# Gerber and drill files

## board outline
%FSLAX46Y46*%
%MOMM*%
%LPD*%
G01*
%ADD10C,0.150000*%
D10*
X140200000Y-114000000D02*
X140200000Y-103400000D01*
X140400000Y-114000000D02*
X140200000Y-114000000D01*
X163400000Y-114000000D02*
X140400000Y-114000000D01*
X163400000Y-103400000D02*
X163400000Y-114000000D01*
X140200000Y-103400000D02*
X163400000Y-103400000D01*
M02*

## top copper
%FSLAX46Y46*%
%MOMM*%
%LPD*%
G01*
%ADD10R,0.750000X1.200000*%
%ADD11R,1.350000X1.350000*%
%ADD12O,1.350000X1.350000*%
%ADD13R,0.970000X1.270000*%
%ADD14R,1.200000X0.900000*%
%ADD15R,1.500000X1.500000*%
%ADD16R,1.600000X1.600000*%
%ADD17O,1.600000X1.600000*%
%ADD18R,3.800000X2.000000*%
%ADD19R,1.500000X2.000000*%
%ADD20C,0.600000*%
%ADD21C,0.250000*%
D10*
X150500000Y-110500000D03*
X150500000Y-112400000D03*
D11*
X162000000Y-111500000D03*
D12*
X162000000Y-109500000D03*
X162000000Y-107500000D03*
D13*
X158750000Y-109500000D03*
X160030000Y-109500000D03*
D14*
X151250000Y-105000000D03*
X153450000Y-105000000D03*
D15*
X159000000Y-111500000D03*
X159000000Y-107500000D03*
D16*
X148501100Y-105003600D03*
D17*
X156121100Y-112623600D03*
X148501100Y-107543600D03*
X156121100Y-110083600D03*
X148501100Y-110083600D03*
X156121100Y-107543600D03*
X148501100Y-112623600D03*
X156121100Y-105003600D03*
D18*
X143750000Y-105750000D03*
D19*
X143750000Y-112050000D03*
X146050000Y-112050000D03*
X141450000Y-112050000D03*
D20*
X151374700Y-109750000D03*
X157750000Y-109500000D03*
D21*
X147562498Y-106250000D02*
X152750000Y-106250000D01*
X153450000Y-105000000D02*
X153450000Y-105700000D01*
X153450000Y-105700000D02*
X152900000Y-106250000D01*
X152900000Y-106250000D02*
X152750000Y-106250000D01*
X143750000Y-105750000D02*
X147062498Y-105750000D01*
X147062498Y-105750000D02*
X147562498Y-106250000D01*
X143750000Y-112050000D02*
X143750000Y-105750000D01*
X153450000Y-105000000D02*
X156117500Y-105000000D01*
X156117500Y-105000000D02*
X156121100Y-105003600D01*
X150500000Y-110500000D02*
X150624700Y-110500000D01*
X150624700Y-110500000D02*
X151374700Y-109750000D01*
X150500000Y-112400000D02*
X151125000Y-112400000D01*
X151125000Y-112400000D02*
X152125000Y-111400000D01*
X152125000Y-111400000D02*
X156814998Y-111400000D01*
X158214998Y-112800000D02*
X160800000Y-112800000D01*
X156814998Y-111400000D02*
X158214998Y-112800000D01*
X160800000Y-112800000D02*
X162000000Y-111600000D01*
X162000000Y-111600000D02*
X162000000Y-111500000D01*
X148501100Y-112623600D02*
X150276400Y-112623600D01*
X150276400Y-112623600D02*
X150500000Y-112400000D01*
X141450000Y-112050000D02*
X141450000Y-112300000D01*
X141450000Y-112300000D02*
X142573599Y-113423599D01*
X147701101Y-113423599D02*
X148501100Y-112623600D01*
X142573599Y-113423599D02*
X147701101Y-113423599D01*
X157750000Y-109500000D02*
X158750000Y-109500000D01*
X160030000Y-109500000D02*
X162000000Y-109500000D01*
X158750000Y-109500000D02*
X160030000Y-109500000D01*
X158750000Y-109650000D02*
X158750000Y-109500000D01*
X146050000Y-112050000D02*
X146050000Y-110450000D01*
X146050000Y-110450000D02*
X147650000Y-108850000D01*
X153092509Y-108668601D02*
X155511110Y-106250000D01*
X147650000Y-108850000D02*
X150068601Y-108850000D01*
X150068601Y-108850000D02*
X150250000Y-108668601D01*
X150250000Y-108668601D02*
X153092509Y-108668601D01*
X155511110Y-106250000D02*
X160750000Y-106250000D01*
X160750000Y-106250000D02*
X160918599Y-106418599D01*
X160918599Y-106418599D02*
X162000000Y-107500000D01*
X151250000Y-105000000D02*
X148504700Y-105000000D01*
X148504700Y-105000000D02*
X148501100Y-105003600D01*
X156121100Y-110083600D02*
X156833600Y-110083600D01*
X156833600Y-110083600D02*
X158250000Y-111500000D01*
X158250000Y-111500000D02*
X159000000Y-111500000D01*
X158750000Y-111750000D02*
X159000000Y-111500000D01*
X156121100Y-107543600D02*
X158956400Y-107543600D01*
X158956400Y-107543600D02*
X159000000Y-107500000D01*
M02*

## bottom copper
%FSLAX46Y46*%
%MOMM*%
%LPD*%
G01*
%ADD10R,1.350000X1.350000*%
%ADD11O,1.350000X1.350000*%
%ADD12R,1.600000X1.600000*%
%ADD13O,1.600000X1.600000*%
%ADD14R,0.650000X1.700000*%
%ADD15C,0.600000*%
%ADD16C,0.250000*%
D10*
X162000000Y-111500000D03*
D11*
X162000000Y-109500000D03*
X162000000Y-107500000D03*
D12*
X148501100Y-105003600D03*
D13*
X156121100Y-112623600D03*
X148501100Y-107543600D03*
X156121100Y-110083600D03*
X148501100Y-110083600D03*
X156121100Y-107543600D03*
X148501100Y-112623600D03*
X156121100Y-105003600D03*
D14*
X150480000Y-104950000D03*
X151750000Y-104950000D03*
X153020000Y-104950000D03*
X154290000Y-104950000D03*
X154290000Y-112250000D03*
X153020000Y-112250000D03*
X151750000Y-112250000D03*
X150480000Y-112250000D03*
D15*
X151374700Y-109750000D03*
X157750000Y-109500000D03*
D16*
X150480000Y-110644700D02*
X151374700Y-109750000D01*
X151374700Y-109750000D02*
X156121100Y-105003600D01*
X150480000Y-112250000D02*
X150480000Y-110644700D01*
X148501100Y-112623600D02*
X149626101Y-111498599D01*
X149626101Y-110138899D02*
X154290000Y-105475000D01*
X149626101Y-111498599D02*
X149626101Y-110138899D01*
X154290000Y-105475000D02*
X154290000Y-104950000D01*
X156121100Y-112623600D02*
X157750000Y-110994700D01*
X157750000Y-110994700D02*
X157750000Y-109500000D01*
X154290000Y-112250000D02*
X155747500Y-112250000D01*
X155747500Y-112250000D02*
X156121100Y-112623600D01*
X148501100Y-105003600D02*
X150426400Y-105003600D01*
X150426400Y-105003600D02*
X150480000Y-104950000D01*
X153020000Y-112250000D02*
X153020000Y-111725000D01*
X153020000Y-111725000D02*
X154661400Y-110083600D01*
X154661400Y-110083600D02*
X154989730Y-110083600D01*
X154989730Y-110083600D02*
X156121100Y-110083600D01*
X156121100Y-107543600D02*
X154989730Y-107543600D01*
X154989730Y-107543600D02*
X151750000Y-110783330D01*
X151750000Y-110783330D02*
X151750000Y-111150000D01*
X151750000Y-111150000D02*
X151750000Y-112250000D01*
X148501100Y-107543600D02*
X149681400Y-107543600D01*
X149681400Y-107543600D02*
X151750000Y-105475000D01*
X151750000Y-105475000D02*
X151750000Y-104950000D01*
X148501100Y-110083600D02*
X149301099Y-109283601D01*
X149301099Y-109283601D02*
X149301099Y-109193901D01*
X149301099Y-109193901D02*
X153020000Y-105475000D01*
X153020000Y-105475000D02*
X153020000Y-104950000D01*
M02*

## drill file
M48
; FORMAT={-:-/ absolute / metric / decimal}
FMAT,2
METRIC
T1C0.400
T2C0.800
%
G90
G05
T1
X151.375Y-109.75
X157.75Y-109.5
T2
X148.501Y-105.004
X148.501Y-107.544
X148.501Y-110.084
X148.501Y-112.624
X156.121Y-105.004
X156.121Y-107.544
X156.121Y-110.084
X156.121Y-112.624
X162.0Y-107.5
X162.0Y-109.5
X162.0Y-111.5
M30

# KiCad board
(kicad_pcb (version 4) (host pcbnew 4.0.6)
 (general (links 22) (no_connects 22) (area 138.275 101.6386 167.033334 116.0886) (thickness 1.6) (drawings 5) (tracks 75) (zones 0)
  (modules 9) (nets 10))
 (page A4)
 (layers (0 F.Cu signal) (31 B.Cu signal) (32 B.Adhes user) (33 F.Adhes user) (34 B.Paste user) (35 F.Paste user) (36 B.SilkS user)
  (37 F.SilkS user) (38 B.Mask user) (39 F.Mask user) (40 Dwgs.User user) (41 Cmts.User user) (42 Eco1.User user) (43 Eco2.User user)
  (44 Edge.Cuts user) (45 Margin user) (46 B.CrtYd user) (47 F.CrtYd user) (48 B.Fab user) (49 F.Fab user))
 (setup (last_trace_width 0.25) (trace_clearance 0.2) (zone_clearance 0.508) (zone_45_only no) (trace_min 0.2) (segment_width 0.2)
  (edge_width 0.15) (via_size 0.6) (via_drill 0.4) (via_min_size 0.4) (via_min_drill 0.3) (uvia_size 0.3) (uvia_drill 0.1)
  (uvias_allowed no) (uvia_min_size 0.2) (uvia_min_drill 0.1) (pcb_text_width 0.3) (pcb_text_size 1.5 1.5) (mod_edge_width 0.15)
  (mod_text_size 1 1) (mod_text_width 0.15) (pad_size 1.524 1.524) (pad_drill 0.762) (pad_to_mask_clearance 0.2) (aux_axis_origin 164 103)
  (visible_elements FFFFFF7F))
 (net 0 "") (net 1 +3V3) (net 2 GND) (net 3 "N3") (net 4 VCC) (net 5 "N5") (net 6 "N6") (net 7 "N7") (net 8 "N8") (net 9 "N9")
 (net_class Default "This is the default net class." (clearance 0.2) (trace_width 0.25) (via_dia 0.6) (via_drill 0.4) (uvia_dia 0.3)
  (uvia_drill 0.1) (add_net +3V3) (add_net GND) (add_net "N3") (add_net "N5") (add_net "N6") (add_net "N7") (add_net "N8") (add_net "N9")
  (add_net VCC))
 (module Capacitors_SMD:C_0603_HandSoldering (layer F.Cu) (at 150.5 111.45 270)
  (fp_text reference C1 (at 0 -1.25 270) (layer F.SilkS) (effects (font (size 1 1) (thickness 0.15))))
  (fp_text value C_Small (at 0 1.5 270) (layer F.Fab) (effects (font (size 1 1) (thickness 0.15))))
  (pad 1 smd rect (at -0.95 0 270) (size 1.2 0.75) (layers F.Cu F.Paste F.Mask) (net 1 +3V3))
  (pad 2 smd rect (at 0.95 0 270) (size 1.2 0.75) (layers F.Cu F.Paste F.Mask) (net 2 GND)))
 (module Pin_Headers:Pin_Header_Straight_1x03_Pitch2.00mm (layer F.Cu) (at 162 111.5 180)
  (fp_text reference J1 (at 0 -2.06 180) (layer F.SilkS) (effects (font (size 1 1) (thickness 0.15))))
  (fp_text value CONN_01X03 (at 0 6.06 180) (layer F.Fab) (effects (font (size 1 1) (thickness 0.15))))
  (pad 1 thru_hole rect (at 0 0 180) (size 1.35 1.35) (drill 0.8) (layers *.Cu *.Mask) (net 2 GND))
  (pad 2 thru_hole oval (at 0 2 180) (size 1.35 1.35) (drill 0.8) (layers *.Cu *.Mask) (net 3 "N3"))
  (pad 3 thru_hole oval (at 0 4 180) (size 1.35 1.35) (drill 0.8) (layers *.Cu *.Mask) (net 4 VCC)))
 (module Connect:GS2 (layer F.Cu) (at 159.39 109.5 90)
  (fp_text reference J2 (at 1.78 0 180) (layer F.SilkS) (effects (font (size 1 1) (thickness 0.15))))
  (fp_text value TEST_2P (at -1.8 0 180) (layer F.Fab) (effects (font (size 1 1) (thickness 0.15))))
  (pad 1 smd rect (at 0 -0.64 90) (size 1.27 0.97) (layers F.Cu F.Paste F.Mask) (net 3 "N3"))
  (pad 2 smd rect (at 0 0.64 90) (size 1.27 0.97) (layers F.Cu F.Paste F.Mask) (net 3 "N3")))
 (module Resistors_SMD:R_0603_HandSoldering (layer F.Cu) (at 152.35 105)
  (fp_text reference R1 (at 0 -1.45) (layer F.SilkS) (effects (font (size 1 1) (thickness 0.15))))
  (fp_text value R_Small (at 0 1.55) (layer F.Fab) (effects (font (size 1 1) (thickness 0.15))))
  (pad 1 smd rect (at -1.1 0) (size 1.2 0.9) (layers F.Cu F.Paste F.Mask) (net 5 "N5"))
  (pad 2 smd rect (at 1.1 0) (size 1.2 0.9) (layers F.Cu F.Paste F.Mask) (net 1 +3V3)))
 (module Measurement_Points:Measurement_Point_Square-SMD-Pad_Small (layer F.Cu) (at 159 111.5)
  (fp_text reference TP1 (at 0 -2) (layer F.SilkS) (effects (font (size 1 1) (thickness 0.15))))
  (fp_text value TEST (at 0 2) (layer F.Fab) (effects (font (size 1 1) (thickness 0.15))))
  (pad 1 smd rect (at 0 0) (size 1.5 1.5) (layers F.Cu F.Mask) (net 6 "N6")))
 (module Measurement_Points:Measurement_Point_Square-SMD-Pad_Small (layer F.Cu) (at 159 107.5)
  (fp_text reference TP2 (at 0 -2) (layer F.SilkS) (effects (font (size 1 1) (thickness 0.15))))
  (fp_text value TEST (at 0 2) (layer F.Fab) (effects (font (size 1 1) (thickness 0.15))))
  (pad 1 smd rect (at 0 0) (size 1.5 1.5) (layers F.Cu F.Mask) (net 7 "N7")))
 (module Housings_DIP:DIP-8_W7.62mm (layer F.Cu) (at 148.5011 105.0036)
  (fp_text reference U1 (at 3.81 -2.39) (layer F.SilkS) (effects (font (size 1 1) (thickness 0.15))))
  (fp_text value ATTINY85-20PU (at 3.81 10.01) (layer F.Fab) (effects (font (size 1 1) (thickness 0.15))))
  (pad 1 thru_hole rect (at 0 0) (size 1.6 1.6) (drill 0.8) (layers *.Cu *.Mask) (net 5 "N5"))
  (pad 5 thru_hole oval (at 7.62 7.62) (size 1.6 1.6) (drill 0.8) (layers *.Cu *.Mask) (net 3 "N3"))
  (pad 2 thru_hole oval (at 0 2.54) (size 1.6 1.6) (drill 0.8) (layers *.Cu *.Mask) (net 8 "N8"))
  (pad 6 thru_hole oval (at 7.62 5.08) (size 1.6 1.6) (drill 0.8) (layers *.Cu *.Mask) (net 6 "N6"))
  (pad 3 thru_hole oval (at 0 5.08) (size 1.6 1.6) (drill 0.8) (layers *.Cu *.Mask) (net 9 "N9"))
  (pad 7 thru_hole oval (at 7.62 2.54) (size 1.6 1.6) (drill 0.8) (layers *.Cu *.Mask) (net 7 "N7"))
  (pad 4 thru_hole oval (at 0 7.62) (size 1.6 1.6) (drill 0.8) (layers *.Cu *.Mask) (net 2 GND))
  (pad 8 thru_hole oval (at 7.62 0) (size 1.6 1.6) (drill 0.8) (layers *.Cu *.Mask) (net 1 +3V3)))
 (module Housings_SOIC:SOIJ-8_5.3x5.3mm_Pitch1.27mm (layer B.Cu) (at 152.385 108.6 270)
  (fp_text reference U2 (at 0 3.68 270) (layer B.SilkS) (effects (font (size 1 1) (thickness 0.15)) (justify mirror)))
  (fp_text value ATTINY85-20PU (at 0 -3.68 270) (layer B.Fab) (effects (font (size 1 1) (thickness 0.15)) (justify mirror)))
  (pad 1 smd rect (at -3.65 1.905 270) (size 1.7 0.65) (layers B.Cu B.Paste B.Mask) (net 5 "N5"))
  (pad 2 smd rect (at -3.65 0.635 270) (size 1.7 0.65) (layers B.Cu B.Paste B.Mask) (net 8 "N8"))
  (pad 3 smd rect (at -3.65 -0.635 270) (size 1.7 0.65) (layers B.Cu B.Paste B.Mask) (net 9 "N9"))
  (pad 4 smd rect (at -3.65 -1.905 270) (size 1.7 0.65) (layers B.Cu B.Paste B.Mask) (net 2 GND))
  (pad 5 smd rect (at 3.65 -1.905 270) (size 1.7 0.65) (layers B.Cu B.Paste B.Mask) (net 3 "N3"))
  (pad 6 smd rect (at 3.65 -0.635 270) (size 1.7 0.65) (layers B.Cu B.Paste B.Mask) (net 6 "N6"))
  (pad 7 smd rect (at 3.65 0.635 270) (size 1.7 0.65) (layers B.Cu B.Paste B.Mask) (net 7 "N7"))
  (pad 8 smd rect (at 3.65 1.905 270) (size 1.7 0.65) (layers B.Cu B.Paste B.Mask) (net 1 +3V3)))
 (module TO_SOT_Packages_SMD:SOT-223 (layer F.Cu) (at 143.75 108.9 90)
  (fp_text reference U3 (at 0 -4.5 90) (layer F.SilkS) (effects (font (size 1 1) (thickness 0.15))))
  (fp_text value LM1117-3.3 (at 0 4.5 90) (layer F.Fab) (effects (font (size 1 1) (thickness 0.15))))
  (pad 4 smd rect (at 3.15 0 90) (size 2 3.8) (layers F.Cu F.Paste F.Mask) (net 1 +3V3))
  (pad 2 smd rect (at -3.15 0 90) (size 2 1.5) (layers F.Cu F.Paste F.Mask) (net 1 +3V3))
  (pad 3 smd rect (at -3.15 2.3 90) (size 2 1.5) (layers F.Cu F.Paste F.Mask) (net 4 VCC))
  (pad 1 smd rect (at -3.15 -2.3 90) (size 2 1.5) (layers F.Cu F.Paste F.Mask) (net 2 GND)))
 (gr_line (start 140.2 114) (end 140.2 103.4) (layer Edge.Cuts) (width 0.15))
 (gr_line (start 140.4 114) (end 140.2 114) (layer Edge.Cuts) (width 0.15))
 (gr_line (start 163.4 114) (end 140.4 114) (layer Edge.Cuts) (width 0.15))
 (gr_line (start 163.4 103.4) (end 163.4 114) (layer Edge.Cuts) (width 0.15))
 (gr_line (start 140.2 103.4) (end 163.4 103.4) (layer Edge.Cuts) (width 0.15))
 (segment (start 147.562498 106.25) (end 152.75 106.25) (width 0.25) (layer F.Cu) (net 1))
 (segment (start 153.45 105) (end 153.45 105.7) (width 0.25) (layer F.Cu) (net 1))
 (segment (start 153.45 105.7) (end 152.9 106.25) (width 0.25) (layer F.Cu) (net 1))
 (segment (start 152.9 106.25) (end 152.75 106.25) (width 0.25) (layer F.Cu) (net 1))
 (segment (start 143.75 105.75) (end 147.062498 105.75) (width 0.25) (layer F.Cu) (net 1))
 (segment (start 147.062498 105.75) (end 147.562498 106.25) (width 0.25) (layer F.Cu) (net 1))
 (segment (start 143.75 112.05) (end 143.75 105.75) (width 0.25) (layer F.Cu) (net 1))
 (segment (start 153.45 105) (end 156.1175 105) (width 0.25) (layer F.Cu) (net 1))
 (segment (start 156.1175 105) (end 156.1211 105.0036) (width 0.25) (layer F.Cu) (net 1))
 (segment (start 150.48 110.6447) (end 151.3747 109.75) (width 0.25) (layer B.Cu) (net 1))
 (segment (start 151.3747 109.75) (end 156.1211 105.0036) (width 0.25) (layer B.Cu) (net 1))
 (segment (start 150.5 110.5) (end 150.6247 110.5) (width 0.25) (layer F.Cu) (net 1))
 (segment (start 150.6247 110.5) (end 151.3747 109.75) (width 0.25) (layer F.Cu) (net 1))
 (via (at 151.3747 109.75) (size 0.6) (drill 0.4) (layers F.Cu B.Cu) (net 1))
 (segment (start 150.48 112.25) (end 150.48 110.6447) (width 0.25) (layer B.Cu) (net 1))
 (segment (start 150.5 112.4) (end 151.125 112.4) (width 0.25) (layer F.Cu) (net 2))
 (segment (start 151.125 112.4) (end 152.125 111.4) (width 0.25) (layer F.Cu) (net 2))
 (segment (start 152.125 111.4) (end 156.814998 111.4) (width 0.25) (layer F.Cu) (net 2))
 (segment (start 158.214998 112.8) (end 160.8 112.8) (width 0.25) (layer F.Cu) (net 2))
 (segment (start 156.814998 111.4) (end 158.214998 112.8) (width 0.25) (layer F.Cu) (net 2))
 (segment (start 160.8 112.8) (end 162 111.6) (width 0.25) (layer F.Cu) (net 2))
 (segment (start 162 111.6) (end 162 111.5) (width 0.25) (layer F.Cu) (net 2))
 (segment (start 148.5011 112.6236) (end 150.2764 112.6236) (width 0.25) (layer F.Cu) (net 2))
 (segment (start 150.2764 112.6236) (end 150.5 112.4) (width 0.25) (layer F.Cu) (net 2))
 (segment (start 141.45 112.05) (end 141.45 112.3) (width 0.25) (layer F.Cu) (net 2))
 (segment (start 141.45 112.3) (end 142.573599 113.423599) (width 0.25) (layer F.Cu) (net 2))
 (segment (start 147.701101 113.423599) (end 148.5011 112.6236) (width 0.25) (layer F.Cu) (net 2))
 (segment (start 142.573599 113.423599) (end 147.701101 113.423599) (width 0.25) (layer F.Cu) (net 2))
 (segment (start 148.5011 112.6236) (end 149.626101 111.498599) (width 0.25) (layer B.Cu) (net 2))
 (segment (start 149.626101 110.138899) (end 154.29 105.475) (width 0.25) (layer B.Cu) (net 2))
 (segment (start 149.626101 111.498599) (end 149.626101 110.138899) (width 0.25) (layer B.Cu) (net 2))
 (segment (start 154.29 105.475) (end 154.29 104.95) (width 0.25) (layer B.Cu) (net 2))
 (segment (start 157.75 109.5) (end 158.75 109.5) (width 0.25) (layer F.Cu) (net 3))
 (segment (start 156.1211 112.6236) (end 157.75 110.9947) (width 0.25) (layer B.Cu) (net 3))
 (segment (start 157.75 110.9947) (end 157.75 109.5) (width 0.25) (layer B.Cu) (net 3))
 (via (at 157.75 109.5) (size 0.6) (drill 0.4) (layers F.Cu B.Cu) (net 3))
 (segment (start 160.03 109.5) (end 162 109.5) (width 0.25) (layer F.Cu) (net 3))
 (segment (start 158.75 109.5) (end 160.03 109.5) (width 0.25) (layer F.Cu) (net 3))
 (segment (start 158.75 109.65) (end 158.75 109.5) (width 0.25) (layer F.Cu) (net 3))
 (segment (start 154.29 112.25) (end 155.7475 112.25) (width 0.25) (layer B.Cu) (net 3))
 (segment (start 155.7475 112.25) (end 156.1211 112.6236) (width 0.25) (layer B.Cu) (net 3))
 (segment (start 146.05 112.05) (end 146.05 110.45) (width 0.25) (layer F.Cu) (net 4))
 (segment (start 146.05 110.45) (end 147.65 108.85) (width 0.25) (layer F.Cu) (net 4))
 (segment (start 153.092509 108.668601) (end 155.51111 106.25) (width 0.25) (layer F.Cu) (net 4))
 (segment (start 147.65 108.85) (end 150.068601 108.85) (width 0.25) (layer F.Cu) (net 4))
 (segment (start 150.068601 108.85) (end 150.25 108.668601) (width 0.25) (layer F.Cu) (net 4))
 (segment (start 150.25 108.668601) (end 153.092509 108.668601) (width 0.25) (layer F.Cu) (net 4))
 (segment (start 155.51111 106.25) (end 160.75 106.25) (width 0.25) (layer F.Cu) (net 4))
 (segment (start 160.75 106.25) (end 160.918599 106.418599) (width 0.25) (layer F.Cu) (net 4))
 (segment (start 160.918599 106.418599) (end 162 107.5) (width 0.25) (layer F.Cu) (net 4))
 (segment (start 151.25 105) (end 148.5047 105) (width 0.25) (layer F.Cu) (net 5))
 (segment (start 148.5047 105) (end 148.5011 105.0036) (width 0.25) (layer F.Cu) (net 5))
 (segment (start 148.5011 105.0036) (end 150.4264 105.0036) (width 0.25) (layer B.Cu) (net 5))
 (segment (start 150.4264 105.0036) (end 150.48 104.95) (width 0.25) (layer B.Cu) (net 5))
 (segment (start 156.1211 110.0836) (end 156.8336 110.0836) (width 0.25) (layer F.Cu) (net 6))
 (segment (start 156.8336 110.0836) (end 158.25 111.5) (width 0.25) (layer F.Cu) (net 6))
 (segment (start 158.25 111.5) (end 159 111.5) (width 0.25) (layer F.Cu) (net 6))
 (segment (start 158.75 111.75) (end 159 111.5) (width 0.25) (layer F.Cu) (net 6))
 (segment (start 153.02 112.25) (end 153.02 111.725) (width 0.25) (layer B.Cu) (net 6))
 (segment (start 153.02 111.725) (end 154.6614 110.0836) (width 0.25) (layer B.Cu) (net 6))
 (segment (start 154.6614 110.0836) (end 154.98973 110.0836) (width 0.25) (layer B.Cu) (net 6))
 (segment (start 154.98973 110.0836) (end 156.1211 110.0836) (width 0.25) (layer B.Cu) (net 6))
 (segment (start 156.1211 107.5436) (end 158.9564 107.5436) (width 0.25) (layer F.Cu) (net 7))
 (segment (start 158.9564 107.5436) (end 159 107.5) (width 0.25) (layer F.Cu) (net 7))
 (segment (start 156.1211 107.5436) (end 154.98973 107.5436) (width 0.25) (layer B.Cu) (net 7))
 (segment (start 154.98973 107.5436) (end 151.75 110.78333) (width 0.25) (layer B.Cu) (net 7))
 (segment (start 151.75 110.78333) (end 151.75 111.15) (width 0.25) (layer B.Cu) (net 7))
 (segment (start 151.75 111.15) (end 151.75 112.25) (width 0.25) (layer B.Cu) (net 7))
 (segment (start 148.5011 107.5436) (end 149.6814 107.5436) (width 0.25) (layer B.Cu) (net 8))
 (segment (start 149.6814 107.5436) (end 151.75 105.475) (width 0.25) (layer B.Cu) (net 8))
 (segment (start 151.75 105.475) (end 151.75 104.95) (width 0.25) (layer B.Cu) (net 8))
 (segment (start 148.5011 110.0836) (end 149.301099 109.283601) (width 0.25) (layer B.Cu) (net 9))
 (segment (start 149.301099 109.283601) (end 149.301099 109.193901) (width 0.25) (layer B.Cu) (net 9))
 (segment (start 149.301099 109.193901) (end 153.02 105.475) (width 0.25) (layer B.Cu) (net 9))
 (segment (start 153.02 105.475) (end 153.02 104.95) (width 0.25) (layer B.Cu) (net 9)))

